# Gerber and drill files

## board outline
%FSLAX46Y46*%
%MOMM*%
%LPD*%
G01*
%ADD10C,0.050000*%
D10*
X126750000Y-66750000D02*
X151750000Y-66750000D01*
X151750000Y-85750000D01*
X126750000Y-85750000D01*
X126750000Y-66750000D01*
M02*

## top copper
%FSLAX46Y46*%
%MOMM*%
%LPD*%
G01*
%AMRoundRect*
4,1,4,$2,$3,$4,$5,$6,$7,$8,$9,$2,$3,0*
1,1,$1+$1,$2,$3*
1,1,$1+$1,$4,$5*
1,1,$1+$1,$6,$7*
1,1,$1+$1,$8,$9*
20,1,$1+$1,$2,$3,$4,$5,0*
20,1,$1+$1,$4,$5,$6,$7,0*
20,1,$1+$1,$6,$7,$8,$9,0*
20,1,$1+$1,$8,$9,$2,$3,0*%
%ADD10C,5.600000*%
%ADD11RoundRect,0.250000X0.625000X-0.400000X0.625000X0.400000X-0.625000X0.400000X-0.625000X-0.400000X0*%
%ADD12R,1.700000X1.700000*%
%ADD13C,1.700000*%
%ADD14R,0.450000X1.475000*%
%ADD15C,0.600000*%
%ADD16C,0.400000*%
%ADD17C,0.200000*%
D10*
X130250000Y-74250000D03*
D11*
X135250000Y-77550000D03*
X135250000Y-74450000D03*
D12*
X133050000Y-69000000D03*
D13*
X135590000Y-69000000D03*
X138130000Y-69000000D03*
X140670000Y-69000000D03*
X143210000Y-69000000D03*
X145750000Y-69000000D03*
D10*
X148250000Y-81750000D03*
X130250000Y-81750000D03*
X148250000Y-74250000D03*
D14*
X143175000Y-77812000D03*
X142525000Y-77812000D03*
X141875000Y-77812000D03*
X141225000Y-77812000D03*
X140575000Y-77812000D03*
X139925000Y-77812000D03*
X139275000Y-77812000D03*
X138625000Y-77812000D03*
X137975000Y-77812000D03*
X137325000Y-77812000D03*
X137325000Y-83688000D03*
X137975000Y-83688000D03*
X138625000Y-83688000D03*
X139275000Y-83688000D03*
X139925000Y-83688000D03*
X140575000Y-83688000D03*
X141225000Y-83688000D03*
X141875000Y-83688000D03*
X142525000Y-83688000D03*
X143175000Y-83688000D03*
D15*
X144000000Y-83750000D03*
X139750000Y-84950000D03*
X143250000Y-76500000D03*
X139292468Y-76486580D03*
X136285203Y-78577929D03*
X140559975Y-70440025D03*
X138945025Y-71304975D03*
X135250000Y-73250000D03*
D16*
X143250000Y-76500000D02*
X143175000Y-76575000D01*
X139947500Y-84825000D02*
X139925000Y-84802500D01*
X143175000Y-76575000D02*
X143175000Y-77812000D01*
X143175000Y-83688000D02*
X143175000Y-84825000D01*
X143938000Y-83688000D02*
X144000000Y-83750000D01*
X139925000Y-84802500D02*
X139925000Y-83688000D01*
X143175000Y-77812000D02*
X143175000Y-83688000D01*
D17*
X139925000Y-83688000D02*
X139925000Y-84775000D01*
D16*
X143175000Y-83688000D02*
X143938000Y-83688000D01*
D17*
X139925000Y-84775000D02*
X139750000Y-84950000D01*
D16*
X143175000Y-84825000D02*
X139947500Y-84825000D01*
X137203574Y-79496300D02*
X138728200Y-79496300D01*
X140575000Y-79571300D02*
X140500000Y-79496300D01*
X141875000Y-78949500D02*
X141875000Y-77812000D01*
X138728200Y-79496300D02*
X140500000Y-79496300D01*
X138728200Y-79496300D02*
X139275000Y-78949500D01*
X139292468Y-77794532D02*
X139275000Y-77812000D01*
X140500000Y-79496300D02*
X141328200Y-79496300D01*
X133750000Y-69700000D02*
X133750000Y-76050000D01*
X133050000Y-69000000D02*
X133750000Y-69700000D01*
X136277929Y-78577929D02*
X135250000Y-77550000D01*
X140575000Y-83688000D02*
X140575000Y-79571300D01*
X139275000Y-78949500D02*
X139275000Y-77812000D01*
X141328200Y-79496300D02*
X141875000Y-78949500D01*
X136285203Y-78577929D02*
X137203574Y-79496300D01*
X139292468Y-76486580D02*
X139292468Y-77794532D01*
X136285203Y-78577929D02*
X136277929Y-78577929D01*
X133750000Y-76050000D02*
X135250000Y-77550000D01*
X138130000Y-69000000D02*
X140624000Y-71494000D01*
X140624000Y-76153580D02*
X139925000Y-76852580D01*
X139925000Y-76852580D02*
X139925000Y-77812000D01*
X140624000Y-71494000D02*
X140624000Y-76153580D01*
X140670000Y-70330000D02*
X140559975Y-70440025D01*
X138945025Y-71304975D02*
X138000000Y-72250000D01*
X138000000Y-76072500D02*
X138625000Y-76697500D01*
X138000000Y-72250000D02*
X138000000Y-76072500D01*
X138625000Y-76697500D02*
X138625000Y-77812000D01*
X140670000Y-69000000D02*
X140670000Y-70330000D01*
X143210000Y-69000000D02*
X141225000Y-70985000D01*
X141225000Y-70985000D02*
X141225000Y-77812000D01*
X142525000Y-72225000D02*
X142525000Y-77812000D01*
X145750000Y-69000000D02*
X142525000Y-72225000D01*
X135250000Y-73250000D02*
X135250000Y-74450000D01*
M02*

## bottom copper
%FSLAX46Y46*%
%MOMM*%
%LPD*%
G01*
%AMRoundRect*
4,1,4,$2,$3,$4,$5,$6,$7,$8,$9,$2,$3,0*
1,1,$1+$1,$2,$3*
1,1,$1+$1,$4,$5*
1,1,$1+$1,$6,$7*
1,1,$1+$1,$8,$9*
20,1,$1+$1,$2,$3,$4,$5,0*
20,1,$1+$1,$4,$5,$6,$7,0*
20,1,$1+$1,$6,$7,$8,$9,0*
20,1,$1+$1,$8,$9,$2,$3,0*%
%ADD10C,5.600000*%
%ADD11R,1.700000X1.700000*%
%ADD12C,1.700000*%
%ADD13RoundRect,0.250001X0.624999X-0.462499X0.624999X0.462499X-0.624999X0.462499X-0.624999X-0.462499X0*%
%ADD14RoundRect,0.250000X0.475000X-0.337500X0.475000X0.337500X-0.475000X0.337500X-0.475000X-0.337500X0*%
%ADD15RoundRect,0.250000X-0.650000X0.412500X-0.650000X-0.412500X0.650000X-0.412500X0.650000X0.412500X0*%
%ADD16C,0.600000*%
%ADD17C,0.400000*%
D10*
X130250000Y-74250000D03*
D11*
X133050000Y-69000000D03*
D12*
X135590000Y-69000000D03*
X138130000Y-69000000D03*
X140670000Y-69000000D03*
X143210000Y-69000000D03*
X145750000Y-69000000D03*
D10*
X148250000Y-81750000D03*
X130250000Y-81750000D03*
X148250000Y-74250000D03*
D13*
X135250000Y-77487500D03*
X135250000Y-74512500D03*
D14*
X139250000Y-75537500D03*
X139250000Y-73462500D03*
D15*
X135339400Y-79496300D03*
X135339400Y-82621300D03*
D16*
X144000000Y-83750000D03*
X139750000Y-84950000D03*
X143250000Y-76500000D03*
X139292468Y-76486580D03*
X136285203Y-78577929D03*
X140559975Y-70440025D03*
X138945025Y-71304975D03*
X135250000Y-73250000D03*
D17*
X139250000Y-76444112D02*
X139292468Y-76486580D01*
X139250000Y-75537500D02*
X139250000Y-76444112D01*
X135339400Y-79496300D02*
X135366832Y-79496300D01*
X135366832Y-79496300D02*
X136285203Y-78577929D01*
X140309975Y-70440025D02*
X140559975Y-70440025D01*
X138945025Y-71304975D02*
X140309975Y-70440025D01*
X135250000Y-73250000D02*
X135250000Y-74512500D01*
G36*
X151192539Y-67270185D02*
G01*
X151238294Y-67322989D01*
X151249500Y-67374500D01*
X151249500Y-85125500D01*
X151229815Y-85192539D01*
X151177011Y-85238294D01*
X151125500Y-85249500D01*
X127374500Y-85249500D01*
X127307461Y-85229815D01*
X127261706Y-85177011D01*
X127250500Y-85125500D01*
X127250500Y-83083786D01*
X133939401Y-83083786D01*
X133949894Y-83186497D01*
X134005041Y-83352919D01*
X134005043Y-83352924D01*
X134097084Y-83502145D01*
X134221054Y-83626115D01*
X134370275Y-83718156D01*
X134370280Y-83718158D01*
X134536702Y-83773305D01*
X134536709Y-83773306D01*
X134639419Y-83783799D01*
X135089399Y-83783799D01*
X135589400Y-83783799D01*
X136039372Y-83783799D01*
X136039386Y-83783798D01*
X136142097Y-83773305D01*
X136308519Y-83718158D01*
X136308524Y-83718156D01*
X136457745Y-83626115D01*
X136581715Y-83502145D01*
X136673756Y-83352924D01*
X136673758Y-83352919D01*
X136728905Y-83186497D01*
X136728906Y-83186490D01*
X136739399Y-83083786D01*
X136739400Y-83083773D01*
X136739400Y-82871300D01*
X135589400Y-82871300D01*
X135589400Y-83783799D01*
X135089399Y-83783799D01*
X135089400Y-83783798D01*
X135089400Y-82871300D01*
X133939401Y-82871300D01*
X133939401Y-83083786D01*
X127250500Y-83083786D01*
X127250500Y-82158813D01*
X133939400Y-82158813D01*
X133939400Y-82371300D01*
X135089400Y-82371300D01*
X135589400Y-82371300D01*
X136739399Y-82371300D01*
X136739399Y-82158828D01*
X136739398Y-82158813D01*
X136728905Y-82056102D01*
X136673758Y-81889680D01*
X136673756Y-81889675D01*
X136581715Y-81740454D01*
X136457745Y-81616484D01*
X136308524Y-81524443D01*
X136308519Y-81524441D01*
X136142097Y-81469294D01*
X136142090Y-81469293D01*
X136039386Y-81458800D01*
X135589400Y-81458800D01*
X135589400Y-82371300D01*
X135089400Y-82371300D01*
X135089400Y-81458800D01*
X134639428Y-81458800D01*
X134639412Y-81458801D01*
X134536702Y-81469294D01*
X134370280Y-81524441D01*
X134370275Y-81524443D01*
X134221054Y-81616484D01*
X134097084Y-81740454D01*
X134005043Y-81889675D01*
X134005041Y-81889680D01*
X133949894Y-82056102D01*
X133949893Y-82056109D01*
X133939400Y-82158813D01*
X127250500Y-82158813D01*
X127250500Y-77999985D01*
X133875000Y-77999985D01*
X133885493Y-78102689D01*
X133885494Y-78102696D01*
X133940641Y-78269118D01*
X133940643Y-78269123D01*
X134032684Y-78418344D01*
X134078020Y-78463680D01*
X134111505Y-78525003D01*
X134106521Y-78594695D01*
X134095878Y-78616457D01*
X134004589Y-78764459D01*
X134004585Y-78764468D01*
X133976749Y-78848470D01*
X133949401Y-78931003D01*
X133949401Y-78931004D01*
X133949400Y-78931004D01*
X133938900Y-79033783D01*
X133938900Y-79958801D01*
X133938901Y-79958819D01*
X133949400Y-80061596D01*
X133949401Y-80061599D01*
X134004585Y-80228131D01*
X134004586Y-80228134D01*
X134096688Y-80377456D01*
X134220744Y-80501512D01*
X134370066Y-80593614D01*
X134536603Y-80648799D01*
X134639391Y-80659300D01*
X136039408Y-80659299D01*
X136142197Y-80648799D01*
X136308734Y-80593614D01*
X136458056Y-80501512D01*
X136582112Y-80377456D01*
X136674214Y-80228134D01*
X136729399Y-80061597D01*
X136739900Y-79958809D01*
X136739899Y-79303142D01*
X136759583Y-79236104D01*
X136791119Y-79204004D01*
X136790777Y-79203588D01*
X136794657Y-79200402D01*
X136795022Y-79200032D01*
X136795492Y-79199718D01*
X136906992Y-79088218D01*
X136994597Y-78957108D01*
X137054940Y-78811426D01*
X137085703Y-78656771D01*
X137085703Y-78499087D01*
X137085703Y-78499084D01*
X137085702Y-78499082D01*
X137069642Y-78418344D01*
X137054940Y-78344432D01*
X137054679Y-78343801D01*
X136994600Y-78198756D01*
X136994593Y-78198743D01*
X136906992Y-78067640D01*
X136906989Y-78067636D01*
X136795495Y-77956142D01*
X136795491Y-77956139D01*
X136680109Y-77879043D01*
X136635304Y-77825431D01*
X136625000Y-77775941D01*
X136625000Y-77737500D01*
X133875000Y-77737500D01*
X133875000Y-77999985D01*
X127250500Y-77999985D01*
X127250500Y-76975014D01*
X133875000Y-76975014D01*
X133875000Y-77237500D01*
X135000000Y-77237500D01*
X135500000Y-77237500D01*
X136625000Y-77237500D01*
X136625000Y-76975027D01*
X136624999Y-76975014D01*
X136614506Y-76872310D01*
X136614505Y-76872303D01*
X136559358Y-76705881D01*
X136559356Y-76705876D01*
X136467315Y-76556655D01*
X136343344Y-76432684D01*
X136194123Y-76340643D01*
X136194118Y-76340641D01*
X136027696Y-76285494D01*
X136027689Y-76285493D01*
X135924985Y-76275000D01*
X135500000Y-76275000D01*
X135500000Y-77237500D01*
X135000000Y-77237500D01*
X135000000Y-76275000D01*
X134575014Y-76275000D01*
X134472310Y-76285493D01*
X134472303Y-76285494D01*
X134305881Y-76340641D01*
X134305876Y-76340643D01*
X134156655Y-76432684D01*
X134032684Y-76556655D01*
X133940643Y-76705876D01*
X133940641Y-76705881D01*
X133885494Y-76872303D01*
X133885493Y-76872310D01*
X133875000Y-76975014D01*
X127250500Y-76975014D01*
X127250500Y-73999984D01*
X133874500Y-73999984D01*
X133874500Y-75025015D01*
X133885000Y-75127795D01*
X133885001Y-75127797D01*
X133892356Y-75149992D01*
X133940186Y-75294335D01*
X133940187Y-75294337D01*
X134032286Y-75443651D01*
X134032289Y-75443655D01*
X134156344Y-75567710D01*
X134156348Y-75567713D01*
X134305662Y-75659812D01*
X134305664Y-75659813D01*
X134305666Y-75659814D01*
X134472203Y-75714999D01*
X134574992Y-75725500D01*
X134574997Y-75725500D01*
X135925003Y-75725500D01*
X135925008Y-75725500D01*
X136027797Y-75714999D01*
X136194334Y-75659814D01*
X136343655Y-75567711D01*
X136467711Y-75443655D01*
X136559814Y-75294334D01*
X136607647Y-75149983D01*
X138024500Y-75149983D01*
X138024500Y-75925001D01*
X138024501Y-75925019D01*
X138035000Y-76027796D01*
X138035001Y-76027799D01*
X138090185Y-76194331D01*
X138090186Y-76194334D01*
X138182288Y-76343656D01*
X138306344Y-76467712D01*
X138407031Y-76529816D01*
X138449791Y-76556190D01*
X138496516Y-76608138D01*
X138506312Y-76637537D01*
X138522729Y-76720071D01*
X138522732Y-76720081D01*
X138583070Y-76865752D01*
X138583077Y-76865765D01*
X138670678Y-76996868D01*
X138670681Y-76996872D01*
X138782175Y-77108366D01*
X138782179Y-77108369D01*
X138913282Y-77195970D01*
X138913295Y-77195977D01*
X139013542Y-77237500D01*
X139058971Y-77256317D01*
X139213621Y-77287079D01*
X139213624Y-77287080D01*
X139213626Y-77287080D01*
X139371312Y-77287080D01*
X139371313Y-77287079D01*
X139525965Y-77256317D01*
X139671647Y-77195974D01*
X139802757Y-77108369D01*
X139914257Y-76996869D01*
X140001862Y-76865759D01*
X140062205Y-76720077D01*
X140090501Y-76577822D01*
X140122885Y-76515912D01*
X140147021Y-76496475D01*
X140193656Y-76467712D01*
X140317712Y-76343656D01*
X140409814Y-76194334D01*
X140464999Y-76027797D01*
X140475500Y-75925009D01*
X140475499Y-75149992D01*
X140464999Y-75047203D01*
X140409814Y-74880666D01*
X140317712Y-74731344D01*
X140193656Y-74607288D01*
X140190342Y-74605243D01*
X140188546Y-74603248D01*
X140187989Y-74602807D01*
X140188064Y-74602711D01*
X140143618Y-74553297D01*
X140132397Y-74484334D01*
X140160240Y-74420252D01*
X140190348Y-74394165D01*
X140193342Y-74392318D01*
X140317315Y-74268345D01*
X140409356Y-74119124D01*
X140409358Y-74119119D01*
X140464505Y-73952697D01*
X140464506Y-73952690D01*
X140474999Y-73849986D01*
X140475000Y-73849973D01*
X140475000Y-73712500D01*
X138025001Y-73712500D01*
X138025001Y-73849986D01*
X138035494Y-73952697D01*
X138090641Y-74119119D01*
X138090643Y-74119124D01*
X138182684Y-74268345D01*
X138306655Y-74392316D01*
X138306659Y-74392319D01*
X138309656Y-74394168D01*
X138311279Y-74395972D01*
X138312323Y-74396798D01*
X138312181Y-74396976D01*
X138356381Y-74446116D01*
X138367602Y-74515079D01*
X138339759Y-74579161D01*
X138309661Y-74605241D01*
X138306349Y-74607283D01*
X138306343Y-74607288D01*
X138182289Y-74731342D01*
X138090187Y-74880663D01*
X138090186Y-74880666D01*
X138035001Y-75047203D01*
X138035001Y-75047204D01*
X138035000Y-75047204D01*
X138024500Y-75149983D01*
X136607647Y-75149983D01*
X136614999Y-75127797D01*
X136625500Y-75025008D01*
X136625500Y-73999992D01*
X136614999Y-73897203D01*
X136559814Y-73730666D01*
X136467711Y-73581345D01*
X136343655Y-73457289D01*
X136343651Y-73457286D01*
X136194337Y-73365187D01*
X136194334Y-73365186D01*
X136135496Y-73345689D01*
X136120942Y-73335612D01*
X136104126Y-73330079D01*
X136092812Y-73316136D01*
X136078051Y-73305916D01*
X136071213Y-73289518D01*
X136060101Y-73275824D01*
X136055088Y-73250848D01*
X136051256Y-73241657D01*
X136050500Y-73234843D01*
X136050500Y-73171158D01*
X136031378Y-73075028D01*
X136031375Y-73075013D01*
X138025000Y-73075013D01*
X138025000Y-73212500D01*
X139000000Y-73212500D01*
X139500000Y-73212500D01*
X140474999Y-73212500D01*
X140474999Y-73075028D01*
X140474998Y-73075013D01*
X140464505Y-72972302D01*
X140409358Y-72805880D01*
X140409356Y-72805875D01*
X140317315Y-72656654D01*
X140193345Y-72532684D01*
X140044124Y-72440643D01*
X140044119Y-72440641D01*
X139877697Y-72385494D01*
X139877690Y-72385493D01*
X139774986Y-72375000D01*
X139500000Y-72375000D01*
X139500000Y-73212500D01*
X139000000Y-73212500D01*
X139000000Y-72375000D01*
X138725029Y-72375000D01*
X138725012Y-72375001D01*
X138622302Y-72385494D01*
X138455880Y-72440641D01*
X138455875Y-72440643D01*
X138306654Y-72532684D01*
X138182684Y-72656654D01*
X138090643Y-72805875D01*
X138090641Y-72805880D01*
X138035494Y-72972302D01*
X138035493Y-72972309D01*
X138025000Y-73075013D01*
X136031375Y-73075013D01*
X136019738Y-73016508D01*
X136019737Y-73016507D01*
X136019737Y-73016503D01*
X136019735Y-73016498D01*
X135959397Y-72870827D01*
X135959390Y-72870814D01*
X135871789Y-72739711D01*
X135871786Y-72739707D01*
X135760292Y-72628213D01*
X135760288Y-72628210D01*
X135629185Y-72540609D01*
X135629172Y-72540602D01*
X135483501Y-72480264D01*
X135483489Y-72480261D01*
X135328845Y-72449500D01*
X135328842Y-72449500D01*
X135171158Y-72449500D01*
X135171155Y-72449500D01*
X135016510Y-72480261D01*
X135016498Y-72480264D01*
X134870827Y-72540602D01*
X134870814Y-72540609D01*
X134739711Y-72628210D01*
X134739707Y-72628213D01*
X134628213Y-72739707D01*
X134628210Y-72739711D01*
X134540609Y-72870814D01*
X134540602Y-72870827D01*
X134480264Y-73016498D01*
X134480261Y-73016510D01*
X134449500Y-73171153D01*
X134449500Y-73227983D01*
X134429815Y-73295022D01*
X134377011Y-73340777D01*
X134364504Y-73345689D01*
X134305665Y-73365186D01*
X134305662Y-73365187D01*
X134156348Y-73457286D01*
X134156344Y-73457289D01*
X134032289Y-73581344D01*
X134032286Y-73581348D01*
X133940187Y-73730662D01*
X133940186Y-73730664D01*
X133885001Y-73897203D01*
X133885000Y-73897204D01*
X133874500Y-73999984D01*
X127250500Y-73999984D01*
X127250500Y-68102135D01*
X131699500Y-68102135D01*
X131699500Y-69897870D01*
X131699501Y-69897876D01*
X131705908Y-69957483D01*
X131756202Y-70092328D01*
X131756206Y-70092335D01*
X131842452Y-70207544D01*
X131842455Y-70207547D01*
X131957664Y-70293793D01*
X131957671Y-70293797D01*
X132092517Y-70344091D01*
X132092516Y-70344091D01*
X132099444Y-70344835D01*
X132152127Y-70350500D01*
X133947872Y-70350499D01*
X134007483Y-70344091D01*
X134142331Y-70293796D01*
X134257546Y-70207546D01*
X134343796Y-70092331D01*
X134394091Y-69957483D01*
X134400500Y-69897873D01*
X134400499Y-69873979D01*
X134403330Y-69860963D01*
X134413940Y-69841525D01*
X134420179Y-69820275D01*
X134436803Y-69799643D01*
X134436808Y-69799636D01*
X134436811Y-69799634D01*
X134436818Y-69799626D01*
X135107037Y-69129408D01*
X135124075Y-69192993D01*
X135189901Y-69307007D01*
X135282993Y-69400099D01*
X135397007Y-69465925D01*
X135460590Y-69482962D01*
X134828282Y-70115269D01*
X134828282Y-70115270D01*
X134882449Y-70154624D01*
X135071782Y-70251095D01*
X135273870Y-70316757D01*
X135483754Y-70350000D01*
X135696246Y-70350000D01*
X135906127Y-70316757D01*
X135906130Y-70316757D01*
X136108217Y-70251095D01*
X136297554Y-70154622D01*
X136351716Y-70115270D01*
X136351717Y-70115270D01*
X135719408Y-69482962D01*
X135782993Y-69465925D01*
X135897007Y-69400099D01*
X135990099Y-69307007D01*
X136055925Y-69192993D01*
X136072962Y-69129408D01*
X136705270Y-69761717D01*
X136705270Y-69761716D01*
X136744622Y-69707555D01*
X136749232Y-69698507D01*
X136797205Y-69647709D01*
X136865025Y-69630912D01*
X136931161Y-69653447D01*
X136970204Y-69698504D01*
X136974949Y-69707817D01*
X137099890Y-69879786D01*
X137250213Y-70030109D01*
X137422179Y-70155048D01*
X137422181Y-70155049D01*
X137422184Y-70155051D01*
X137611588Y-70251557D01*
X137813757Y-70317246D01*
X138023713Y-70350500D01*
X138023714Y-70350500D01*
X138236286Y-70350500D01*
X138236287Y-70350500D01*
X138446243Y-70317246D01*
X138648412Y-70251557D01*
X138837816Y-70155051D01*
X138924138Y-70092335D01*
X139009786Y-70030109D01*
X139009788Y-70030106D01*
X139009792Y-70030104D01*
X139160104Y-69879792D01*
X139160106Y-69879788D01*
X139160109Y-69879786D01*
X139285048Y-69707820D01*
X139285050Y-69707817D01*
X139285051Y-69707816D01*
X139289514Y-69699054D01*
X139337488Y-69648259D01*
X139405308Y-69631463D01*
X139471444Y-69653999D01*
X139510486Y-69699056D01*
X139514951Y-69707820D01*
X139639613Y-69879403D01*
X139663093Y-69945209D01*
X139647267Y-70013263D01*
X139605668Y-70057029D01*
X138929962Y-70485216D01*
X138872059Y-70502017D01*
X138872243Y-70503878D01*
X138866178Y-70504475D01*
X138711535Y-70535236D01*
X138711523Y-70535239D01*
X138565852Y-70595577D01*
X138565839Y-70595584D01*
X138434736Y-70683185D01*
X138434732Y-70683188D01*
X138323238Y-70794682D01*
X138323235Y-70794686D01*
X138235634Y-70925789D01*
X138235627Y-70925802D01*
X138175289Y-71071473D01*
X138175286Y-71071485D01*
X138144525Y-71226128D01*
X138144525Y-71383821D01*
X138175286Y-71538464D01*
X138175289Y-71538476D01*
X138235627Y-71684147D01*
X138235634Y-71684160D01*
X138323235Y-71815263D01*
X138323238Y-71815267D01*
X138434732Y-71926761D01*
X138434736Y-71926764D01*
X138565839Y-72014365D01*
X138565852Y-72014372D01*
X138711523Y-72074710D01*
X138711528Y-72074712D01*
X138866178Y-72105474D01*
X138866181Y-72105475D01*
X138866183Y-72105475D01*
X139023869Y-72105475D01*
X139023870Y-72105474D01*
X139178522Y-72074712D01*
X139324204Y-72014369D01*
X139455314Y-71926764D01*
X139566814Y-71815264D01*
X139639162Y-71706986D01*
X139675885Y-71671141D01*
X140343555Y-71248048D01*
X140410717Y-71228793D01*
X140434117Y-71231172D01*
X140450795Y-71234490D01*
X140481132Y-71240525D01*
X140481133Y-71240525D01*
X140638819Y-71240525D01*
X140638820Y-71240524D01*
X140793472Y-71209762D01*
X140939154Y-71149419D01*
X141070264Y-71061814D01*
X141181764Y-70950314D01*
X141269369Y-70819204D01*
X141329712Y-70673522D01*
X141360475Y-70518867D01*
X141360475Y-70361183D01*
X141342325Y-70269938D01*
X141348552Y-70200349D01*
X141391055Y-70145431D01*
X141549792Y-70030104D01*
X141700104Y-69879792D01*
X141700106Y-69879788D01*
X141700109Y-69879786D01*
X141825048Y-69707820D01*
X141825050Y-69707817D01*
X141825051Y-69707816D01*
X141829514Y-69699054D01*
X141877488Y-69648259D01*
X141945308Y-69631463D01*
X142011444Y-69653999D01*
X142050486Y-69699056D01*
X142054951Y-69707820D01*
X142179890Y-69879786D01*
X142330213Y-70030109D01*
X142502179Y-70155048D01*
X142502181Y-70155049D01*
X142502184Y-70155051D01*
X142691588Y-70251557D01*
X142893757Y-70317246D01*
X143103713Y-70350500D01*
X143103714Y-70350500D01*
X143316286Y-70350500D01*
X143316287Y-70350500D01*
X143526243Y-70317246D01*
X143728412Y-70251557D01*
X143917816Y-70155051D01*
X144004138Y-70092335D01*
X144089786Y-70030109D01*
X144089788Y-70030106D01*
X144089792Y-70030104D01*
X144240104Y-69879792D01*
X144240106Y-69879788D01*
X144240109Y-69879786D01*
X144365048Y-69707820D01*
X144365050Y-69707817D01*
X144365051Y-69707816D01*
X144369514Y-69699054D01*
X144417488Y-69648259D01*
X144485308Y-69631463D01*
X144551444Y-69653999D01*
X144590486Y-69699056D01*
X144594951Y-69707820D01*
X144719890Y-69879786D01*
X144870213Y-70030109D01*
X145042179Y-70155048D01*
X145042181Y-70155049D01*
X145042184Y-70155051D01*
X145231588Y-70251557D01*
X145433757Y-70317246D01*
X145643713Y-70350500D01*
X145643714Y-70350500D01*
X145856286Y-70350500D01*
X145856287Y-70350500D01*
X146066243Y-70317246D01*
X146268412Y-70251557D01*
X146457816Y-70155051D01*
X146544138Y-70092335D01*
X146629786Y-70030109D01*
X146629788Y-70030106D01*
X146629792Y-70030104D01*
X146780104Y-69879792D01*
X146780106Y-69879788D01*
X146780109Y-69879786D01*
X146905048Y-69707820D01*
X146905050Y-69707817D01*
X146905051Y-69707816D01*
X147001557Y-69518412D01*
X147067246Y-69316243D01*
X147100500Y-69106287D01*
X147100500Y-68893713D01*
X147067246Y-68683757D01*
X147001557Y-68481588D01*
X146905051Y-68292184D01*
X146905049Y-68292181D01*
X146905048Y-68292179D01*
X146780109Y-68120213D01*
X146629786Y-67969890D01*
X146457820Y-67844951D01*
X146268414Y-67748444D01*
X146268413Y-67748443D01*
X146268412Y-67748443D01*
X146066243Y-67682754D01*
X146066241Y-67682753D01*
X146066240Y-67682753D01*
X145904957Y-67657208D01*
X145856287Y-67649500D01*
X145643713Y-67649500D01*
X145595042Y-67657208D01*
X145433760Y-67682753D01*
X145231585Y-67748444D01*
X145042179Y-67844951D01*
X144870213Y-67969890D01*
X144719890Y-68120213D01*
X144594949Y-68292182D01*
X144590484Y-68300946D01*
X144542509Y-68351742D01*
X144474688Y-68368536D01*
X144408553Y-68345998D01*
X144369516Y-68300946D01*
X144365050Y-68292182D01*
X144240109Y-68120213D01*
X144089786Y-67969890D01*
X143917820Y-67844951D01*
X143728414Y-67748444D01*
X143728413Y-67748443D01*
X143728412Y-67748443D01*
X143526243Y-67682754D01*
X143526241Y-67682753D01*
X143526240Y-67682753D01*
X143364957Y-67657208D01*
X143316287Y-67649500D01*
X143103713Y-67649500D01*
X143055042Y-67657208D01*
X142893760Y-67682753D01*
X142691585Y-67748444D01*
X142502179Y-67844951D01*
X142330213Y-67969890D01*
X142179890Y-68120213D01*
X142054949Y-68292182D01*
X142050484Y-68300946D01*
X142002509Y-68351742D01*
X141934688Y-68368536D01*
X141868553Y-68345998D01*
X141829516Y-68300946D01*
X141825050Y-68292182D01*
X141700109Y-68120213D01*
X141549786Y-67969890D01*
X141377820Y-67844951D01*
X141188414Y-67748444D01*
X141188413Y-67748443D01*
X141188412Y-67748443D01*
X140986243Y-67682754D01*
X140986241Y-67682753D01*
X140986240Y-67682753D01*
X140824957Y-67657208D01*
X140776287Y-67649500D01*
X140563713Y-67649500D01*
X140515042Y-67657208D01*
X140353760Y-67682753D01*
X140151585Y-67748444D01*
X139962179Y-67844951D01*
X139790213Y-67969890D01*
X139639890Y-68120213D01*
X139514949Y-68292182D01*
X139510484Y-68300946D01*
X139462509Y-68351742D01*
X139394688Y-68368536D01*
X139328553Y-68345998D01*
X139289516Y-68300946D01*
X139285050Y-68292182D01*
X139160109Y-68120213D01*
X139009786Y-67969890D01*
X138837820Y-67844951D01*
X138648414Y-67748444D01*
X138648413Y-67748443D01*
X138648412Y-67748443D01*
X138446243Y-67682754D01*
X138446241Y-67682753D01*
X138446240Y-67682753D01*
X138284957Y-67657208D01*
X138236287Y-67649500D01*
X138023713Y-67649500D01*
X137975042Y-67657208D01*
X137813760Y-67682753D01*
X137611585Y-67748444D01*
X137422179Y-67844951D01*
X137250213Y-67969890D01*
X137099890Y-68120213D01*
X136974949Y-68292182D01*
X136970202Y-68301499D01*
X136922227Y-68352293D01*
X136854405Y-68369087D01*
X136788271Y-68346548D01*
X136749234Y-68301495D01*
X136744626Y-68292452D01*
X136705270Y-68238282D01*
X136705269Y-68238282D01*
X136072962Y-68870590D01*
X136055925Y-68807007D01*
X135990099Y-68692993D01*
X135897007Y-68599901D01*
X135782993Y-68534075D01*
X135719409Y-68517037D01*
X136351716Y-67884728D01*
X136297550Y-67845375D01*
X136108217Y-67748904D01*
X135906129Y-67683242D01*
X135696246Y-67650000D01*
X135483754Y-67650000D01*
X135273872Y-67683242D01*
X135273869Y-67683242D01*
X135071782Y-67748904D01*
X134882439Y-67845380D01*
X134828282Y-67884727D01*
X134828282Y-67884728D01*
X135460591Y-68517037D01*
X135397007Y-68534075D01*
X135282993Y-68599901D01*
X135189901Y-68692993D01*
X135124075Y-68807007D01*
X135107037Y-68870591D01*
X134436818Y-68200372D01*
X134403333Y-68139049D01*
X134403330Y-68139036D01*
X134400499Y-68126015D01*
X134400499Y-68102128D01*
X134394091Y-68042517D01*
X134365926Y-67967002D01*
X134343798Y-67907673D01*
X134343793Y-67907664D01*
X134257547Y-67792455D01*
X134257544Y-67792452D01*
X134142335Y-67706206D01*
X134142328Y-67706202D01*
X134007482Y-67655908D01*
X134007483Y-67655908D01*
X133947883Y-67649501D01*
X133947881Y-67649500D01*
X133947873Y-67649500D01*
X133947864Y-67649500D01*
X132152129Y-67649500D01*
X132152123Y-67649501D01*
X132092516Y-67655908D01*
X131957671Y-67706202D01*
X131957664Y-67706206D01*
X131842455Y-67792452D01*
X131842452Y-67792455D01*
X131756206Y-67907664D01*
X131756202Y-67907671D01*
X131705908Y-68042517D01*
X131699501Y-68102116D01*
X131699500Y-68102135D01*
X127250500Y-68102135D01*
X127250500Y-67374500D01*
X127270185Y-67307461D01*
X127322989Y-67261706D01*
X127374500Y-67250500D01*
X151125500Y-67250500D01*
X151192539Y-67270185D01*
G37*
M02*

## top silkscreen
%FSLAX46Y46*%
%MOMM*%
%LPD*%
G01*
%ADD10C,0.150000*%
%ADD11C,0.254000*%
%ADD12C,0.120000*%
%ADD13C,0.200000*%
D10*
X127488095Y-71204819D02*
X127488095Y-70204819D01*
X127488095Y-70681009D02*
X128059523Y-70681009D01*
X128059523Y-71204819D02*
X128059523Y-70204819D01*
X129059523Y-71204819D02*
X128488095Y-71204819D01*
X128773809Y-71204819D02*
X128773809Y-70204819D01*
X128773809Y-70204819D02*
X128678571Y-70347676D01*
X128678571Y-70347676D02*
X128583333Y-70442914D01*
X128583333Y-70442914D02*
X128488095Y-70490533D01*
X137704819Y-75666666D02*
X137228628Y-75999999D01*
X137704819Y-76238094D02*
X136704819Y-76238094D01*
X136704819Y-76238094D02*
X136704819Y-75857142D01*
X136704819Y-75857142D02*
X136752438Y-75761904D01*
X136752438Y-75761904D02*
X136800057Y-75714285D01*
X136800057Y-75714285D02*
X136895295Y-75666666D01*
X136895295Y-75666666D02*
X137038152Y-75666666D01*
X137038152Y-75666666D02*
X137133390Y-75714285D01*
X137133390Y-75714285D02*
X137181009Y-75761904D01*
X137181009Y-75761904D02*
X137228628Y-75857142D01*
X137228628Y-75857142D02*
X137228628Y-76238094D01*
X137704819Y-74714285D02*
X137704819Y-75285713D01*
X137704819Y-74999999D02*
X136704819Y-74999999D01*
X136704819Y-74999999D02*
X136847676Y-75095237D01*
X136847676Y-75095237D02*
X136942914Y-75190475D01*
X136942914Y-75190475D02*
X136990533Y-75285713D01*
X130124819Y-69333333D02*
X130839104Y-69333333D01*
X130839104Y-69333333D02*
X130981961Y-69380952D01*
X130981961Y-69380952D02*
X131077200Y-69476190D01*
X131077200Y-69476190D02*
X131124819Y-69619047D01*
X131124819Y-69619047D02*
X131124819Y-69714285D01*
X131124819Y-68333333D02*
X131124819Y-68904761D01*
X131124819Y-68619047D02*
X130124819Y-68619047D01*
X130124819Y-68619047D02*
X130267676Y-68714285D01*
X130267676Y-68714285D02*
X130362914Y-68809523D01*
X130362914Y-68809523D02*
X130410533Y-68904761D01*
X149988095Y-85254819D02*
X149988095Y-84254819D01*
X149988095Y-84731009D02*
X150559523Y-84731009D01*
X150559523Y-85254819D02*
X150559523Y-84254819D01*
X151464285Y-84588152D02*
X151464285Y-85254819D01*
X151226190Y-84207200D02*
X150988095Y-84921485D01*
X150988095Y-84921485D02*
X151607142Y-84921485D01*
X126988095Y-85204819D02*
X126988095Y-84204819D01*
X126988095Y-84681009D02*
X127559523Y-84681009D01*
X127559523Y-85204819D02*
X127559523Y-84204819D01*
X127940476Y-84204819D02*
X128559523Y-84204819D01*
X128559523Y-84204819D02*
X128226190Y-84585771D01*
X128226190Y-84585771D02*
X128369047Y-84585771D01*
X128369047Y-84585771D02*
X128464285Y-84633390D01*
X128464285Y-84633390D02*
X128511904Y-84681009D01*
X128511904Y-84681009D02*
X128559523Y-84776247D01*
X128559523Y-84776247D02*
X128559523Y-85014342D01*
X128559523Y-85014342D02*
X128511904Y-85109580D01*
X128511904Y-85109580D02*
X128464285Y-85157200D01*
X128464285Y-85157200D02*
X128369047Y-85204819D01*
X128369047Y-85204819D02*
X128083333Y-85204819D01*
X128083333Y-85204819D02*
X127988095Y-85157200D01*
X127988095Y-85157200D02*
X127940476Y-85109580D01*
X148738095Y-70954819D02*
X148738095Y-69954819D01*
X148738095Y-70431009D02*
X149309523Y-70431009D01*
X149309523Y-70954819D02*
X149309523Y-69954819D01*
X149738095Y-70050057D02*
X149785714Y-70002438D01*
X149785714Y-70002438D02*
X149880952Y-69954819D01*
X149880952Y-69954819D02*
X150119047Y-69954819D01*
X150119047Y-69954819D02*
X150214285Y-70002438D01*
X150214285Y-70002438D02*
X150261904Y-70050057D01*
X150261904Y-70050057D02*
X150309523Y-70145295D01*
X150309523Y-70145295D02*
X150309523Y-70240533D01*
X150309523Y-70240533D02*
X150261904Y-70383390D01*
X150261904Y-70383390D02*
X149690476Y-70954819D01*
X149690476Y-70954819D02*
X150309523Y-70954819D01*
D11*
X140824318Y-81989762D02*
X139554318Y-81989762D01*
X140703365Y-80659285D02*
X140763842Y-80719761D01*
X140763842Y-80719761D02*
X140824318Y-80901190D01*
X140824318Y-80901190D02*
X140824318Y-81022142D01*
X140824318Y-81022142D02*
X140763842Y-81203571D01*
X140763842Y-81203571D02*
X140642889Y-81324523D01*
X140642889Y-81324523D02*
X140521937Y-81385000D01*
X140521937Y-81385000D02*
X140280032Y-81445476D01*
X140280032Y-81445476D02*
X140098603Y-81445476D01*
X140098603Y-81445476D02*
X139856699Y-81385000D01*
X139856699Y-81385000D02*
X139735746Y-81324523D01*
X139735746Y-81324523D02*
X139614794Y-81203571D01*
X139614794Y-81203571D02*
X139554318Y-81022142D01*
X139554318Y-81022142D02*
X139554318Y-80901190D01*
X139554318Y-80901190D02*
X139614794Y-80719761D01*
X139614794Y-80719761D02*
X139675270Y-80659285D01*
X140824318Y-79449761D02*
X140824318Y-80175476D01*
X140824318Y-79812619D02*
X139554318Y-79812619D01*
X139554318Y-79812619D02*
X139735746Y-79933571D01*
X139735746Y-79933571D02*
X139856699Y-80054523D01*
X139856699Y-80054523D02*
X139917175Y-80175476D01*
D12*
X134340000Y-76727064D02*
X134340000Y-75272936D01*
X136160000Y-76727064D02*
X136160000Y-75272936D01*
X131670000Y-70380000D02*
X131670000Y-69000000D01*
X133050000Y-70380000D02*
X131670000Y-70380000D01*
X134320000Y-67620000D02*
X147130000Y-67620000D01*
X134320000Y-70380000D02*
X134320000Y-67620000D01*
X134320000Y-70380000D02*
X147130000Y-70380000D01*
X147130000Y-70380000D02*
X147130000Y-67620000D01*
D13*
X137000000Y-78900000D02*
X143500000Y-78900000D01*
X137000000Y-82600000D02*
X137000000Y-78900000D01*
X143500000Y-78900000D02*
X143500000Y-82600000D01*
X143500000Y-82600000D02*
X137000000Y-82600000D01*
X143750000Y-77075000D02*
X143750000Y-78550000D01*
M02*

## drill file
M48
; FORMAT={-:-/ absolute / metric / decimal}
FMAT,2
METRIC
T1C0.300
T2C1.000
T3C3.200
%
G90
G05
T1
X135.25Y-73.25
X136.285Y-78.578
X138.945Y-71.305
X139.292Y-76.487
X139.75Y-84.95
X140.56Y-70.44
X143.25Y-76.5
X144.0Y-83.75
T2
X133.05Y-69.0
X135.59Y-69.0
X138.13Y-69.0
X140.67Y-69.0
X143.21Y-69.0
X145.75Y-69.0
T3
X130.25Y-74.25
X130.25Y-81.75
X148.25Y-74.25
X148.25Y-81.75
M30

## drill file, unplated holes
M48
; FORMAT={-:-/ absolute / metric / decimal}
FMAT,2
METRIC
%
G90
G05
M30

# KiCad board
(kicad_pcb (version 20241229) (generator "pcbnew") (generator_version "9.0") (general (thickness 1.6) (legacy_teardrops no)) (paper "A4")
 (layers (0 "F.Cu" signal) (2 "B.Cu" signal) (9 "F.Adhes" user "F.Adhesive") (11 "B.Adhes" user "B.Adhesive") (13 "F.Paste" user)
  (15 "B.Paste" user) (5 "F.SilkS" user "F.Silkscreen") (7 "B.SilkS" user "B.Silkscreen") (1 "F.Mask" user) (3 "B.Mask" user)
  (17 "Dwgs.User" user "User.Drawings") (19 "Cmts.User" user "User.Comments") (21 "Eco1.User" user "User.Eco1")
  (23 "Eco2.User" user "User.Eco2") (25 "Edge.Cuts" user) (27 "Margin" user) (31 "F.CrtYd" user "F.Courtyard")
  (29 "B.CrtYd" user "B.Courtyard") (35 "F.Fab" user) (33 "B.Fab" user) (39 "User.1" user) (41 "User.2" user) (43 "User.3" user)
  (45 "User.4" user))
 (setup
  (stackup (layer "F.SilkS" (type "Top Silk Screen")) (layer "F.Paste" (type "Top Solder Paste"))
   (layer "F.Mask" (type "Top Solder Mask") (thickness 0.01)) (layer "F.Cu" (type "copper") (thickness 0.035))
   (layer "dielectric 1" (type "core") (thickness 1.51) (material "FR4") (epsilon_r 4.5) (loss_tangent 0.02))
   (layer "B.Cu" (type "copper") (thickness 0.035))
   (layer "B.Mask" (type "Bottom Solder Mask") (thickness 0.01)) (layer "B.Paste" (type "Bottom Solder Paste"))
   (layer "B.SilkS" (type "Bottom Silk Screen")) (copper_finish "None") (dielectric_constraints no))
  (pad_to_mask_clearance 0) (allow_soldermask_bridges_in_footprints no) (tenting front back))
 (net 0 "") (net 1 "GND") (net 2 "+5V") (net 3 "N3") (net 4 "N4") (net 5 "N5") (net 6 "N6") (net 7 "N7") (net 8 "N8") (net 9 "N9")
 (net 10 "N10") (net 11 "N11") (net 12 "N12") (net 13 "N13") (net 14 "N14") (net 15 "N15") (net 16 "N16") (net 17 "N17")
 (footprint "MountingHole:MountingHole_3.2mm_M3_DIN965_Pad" (layer "F.Cu") (at 130.25 74.25)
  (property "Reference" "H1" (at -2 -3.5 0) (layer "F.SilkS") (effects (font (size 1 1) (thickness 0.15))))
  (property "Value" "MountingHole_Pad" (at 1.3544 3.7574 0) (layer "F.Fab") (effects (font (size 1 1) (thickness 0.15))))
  (pad "1" thru_hole circle (at 0 0) (size 5.6 5.6) (drill 3.2) (layers "*.Cu" "*.Mask") (remove_unused_layers no) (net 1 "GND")
   (zone_connect 2)))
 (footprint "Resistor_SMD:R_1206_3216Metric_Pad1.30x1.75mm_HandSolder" (layer "F.Cu") (at 135.25 76 90)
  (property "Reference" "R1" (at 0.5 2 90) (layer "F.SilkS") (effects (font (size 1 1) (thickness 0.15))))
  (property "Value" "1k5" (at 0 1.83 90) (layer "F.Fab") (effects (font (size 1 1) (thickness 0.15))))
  (fp_line (start -0.727064 -0.91) (end 0.727064 -0.91) (stroke (width 0.12) (type solid)) (layer "F.SilkS"))
  (fp_line (start -0.727064 0.91) (end 0.727064 0.91) (stroke (width 0.12) (type solid)) (layer "F.SilkS"))
  (pad "1" smd roundrect (at -1.55 0 90) (size 1.3 1.75) (layers "F.Cu" "F.Mask" "F.Paste") (roundrect_rratio 0.192308) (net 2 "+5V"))
  (pad "2" smd roundrect (at 1.55 0 90) (size 1.3 1.75) (layers "F.Cu" "F.Mask" "F.Paste") (roundrect_rratio 0.192308) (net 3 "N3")))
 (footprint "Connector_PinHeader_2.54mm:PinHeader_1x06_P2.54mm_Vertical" (layer "F.Cu") (at 133.05 69 90)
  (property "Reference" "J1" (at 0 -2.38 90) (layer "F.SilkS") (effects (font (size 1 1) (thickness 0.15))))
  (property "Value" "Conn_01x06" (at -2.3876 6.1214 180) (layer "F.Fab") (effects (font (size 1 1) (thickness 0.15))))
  (fp_line (start -1.38 -1.38) (end 0 -1.38) (stroke (width 0.12) (type solid)) (layer "F.SilkS"))
  (fp_line (start -1.38 0) (end -1.38 -1.38) (stroke (width 0.12) (type solid)) (layer "F.SilkS"))
  (fp_line (start 1.38 1.27) (end 1.38 14.08) (stroke (width 0.12) (type solid)) (layer "F.SilkS"))
  (fp_line (start -1.38 1.27) (end 1.38 1.27) (stroke (width 0.12) (type solid)) (layer "F.SilkS"))
  (fp_line (start -1.38 1.27) (end -1.38 14.08) (stroke (width 0.12) (type solid)) (layer "F.SilkS"))
  (fp_line (start -1.38 14.08) (end 1.38 14.08) (stroke (width 0.12) (type solid)) (layer "F.SilkS"))
  (pad "1" thru_hole rect (at 0 0 90) (size 1.7 1.7) (drill 1) (layers "*.Cu" "*.Mask") (remove_unused_layers no) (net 2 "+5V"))
  (pad "2" thru_hole circle (at 0 2.54 90) (size 1.7 1.7) (drill 1) (layers "*.Cu" "*.Mask") (remove_unused_layers no) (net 1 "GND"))
  (pad "3" thru_hole circle (at 0 5.08 90) (size 1.7 1.7) (drill 1) (layers "*.Cu" "*.Mask") (remove_unused_layers no) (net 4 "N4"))
  (pad "4" thru_hole circle (at 0 7.62 90) (size 1.7 1.7) (drill 1) (layers "*.Cu" "*.Mask") (remove_unused_layers no) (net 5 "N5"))
  (pad "5" thru_hole circle (at 0 10.16 90) (size 1.7 1.7) (drill 1) (layers "*.Cu" "*.Mask") (remove_unused_layers no) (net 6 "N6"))
  (pad "6" thru_hole circle (at 0 12.7 90) (size 1.7 1.7) (drill 1) (layers "*.Cu" "*.Mask") (remove_unused_layers no) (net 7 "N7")))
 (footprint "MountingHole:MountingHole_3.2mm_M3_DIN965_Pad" (layer "F.Cu") (at 148.25 81.75)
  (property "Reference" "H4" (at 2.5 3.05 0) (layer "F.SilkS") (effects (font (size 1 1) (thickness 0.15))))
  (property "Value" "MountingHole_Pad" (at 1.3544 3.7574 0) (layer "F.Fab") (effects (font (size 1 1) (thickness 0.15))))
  (pad "1" thru_hole circle (at 0 0) (size 5.6 5.6) (drill 3.2) (layers "*.Cu" "*.Mask") (remove_unused_layers no) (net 1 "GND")
   (zone_connect 2)))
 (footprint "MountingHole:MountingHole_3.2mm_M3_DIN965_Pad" (layer "F.Cu") (at 130.25 81.75)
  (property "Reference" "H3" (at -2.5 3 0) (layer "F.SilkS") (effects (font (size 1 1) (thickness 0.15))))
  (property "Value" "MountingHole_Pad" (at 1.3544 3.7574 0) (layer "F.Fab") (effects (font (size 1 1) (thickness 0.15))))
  (pad "1" thru_hole circle (at 0 0) (size 5.6 5.6) (drill 3.2) (layers "*.Cu" "*.Mask") (remove_unused_layers no) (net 1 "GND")
   (zone_connect 2)))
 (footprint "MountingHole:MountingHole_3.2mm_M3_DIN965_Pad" (layer "F.Cu") (at 148.25 74.25)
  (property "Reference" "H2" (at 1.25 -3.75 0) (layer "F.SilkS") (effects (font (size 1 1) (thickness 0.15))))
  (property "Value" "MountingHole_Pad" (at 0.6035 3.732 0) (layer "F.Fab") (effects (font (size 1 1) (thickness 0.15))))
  (pad "1" thru_hole circle (at 0 0) (size 5.6 5.6) (drill 3.2) (layers "*.Cu" "*.Mask") (remove_unused_layers no) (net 1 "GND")
   (zone_connect 2)))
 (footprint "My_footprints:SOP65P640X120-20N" (layer "F.Cu") (at 140.25 80.75 -90)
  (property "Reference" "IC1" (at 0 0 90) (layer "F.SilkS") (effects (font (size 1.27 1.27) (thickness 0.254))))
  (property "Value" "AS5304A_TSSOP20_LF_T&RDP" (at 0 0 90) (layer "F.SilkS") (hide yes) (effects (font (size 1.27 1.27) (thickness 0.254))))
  (fp_line (start -1.85 3.25) (end -1.85 -3.25) (stroke (width 0.2) (type solid)) (layer "F.SilkS"))
  (fp_line (start 1.85 3.25) (end -1.85 3.25) (stroke (width 0.2) (type solid)) (layer "F.SilkS"))
  (fp_line (start -1.85 -3.25) (end 1.85 -3.25) (stroke (width 0.2) (type solid)) (layer "F.SilkS"))
  (fp_line (start 1.85 -3.25) (end 1.85 3.25) (stroke (width 0.2) (type solid)) (layer "F.SilkS"))
  (fp_line (start -3.675 -3.5) (end -2.2 -3.5) (stroke (width 0.2) (type solid)) (layer "F.SilkS"))
  (pad "1" smd rect (at -2.938 -2.925) (size 0.45 1.475) (layers "F.Cu" "F.Mask" "F.Paste") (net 1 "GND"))
  (pad "2" smd rect (at -2.938 -2.275) (size 0.45 1.475) (layers "F.Cu" "F.Mask" "F.Paste") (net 7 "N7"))
  (pad "3" smd rect (at -2.938 -1.625) (size 0.45 1.475) (layers "F.Cu" "F.Mask" "F.Paste") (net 2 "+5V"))
  (pad "4" smd rect (at -2.938 -0.975) (size 0.45 1.475) (layers "F.Cu" "F.Mask" "F.Paste") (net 6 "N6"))
  (pad "5" smd rect (at -2.938 -0.325) (size 0.45 1.475) (layers "F.Cu" "F.Mask" "F.Paste") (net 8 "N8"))
  (pad "6" smd rect (at -2.938 0.325) (size 0.45 1.475) (layers "F.Cu" "F.Mask" "F.Paste") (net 4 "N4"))
  (pad "7" smd rect (at -2.938 0.975) (size 0.45 1.475) (layers "F.Cu" "F.Mask" "F.Paste") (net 2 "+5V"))
  (pad "8" smd rect (at -2.938 1.625) (size 0.45 1.475) (layers "F.Cu" "F.Mask" "F.Paste") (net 5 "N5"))
  (pad "9" smd rect (at -2.938 2.275) (size 0.45 1.475) (layers "F.Cu" "F.Mask" "F.Paste") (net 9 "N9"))
  (pad "10" smd rect (at -2.938 2.925) (size 0.45 1.475) (layers "F.Cu" "F.Mask" "F.Paste") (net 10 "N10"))
  (pad "11" smd rect (at 2.938 2.925) (size 0.45 1.475) (layers "F.Cu" "F.Mask" "F.Paste") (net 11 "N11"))
  (pad "12" smd rect (at 2.938 2.275) (size 0.45 1.475) (layers "F.Cu" "F.Mask" "F.Paste") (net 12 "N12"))
  (pad "13" smd rect (at 2.938 1.625) (size 0.45 1.475) (layers "F.Cu" "F.Mask" "F.Paste") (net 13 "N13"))
  (pad "14" smd rect (at 2.938 0.975) (size 0.45 1.475) (layers "F.Cu" "F.Mask" "F.Paste") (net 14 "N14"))
  (pad "15" smd rect (at 2.938 0.325) (size 0.45 1.475) (layers "F.Cu" "F.Mask" "F.Paste") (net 1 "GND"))
  (pad "16" smd rect (at 2.938 -0.325) (size 0.45 1.475) (layers "F.Cu" "F.Mask" "F.Paste") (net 2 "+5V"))
  (pad "17" smd rect (at 2.938 -0.975) (size 0.45 1.475) (layers "F.Cu" "F.Mask" "F.Paste") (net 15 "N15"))
  (pad "18" smd rect (at 2.938 -1.625) (size 0.45 1.475) (layers "F.Cu" "F.Mask" "F.Paste") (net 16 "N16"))
  (pad "19" smd rect (at 2.938 -2.275) (size 0.45 1.475) (layers "F.Cu" "F.Mask" "F.Paste") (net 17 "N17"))
  (pad "20" smd rect (at 2.938 -2.925) (size 0.45 1.475) (layers "F.Cu" "F.Mask" "F.Paste") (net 1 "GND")))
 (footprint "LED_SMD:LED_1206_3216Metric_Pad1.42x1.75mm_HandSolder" (layer "B.Cu") (at 135.25 76 90)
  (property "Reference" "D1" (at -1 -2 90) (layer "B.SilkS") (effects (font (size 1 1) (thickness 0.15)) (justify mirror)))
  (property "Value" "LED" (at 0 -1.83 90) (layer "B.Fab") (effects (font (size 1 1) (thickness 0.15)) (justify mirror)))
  (pad "1" smd roundrect (at -1.4875 0 90) (size 1.425 1.75) (layers "B.Cu" "B.Mask" "B.Paste") (roundrect_rratio 0.175439) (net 1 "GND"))
  (pad "2" smd roundrect (at 1.4875 0 90) (size 1.425 1.75) (layers "B.Cu" "B.Mask" "B.Paste") (roundrect_rratio 0.175439) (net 3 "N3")))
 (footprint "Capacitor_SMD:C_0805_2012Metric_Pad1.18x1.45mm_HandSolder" (layer "B.Cu") (at 139.25 74.5 90)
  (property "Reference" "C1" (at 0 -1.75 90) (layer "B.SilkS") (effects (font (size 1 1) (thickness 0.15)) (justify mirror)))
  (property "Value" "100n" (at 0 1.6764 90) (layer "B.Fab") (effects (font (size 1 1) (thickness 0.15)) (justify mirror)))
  (pad "1" smd roundrect (at -1.0375 0 90) (size 1.175 1.45) (layers "B.Cu" "B.Mask" "B.Paste") (roundrect_rratio 0.212766) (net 2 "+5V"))
  (pad "2" smd roundrect (at 1.0375 0 90) (size 1.175 1.45) (layers "B.Cu" "B.Mask" "B.Paste") (roundrect_rratio 0.212766) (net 1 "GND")))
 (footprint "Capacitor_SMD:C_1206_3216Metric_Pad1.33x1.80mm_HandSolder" (layer "B.Cu") (at 135.3394 81.0588 -90)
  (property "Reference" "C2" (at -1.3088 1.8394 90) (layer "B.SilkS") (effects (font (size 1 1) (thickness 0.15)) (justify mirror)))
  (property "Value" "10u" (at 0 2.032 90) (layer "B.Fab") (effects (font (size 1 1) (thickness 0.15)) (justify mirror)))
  (pad "1" smd roundrect (at -1.5625 0 270) (size 1.325 1.8) (layers "B.Cu" "B.Mask" "B.Paste") (roundrect_rratio 0.188679) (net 2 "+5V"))
  (pad "2" smd roundrect (at 1.5625 0 270) (size 1.325 1.8) (layers "B.Cu" "B.Mask" "B.Paste") (roundrect_rratio 0.188679) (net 1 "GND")))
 (gr_rect (start 126.75 66.75) (end 151.75 85.75) (stroke (width 0.05) (type default)) (fill no) (layer "Edge.Cuts"))
 (segment (start 143.25 76.5) (end 143.175 76.575) (width 0.4) (layer "F.Cu") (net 1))
 (segment (start 139.9475 84.825) (end 139.925 84.8025) (width 0.4) (layer "F.Cu") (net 1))
 (segment (start 143.175 76.575) (end 143.175 77.812) (width 0.4) (layer "F.Cu") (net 1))
 (segment (start 143.175 83.688) (end 143.175 84.825) (width 0.4) (layer "F.Cu") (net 1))
 (segment (start 143.938 83.688) (end 144 83.75) (width 0.4) (layer "F.Cu") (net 1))
 (segment (start 139.925 84.8025) (end 139.925 83.688) (width 0.4) (layer "F.Cu") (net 1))
 (segment (start 143.175 77.812) (end 143.175 83.688) (width 0.4) (layer "F.Cu") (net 1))
 (segment (start 139.925 83.688) (end 139.925 84.775) (width 0.2) (layer "F.Cu") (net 1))
 (segment (start 143.175 83.688) (end 143.938 83.688) (width 0.4) (layer "F.Cu") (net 1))
 (segment (start 139.925 84.775) (end 139.75 84.95) (width 0.2) (layer "F.Cu") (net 1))
 (segment (start 143.175 84.825) (end 139.9475 84.825) (width 0.4) (layer "F.Cu") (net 1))
 (via (at 144 83.75) (size 0.6) (drill 0.3) (layers "F.Cu" "B.Cu") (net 1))
 (via (at 139.75 84.95) (size 0.6) (drill 0.3) (layers "F.Cu" "B.Cu") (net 1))
 (via (at 143.25 76.5) (size 0.6) (drill 0.3) (layers "F.Cu" "B.Cu") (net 1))
 (segment (start 137.203574 79.4963) (end 138.7282 79.4963) (width 0.4) (layer "F.Cu") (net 2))
 (segment (start 140.575 79.5713) (end 140.5 79.4963) (width 0.4) (layer "F.Cu") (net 2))
 (segment (start 141.875 78.9495) (end 141.875 77.812) (width 0.4) (layer "F.Cu") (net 2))
 (segment (start 138.7282 79.4963) (end 140.5 79.4963) (width 0.4) (layer "F.Cu") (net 2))
 (segment (start 138.7282 79.4963) (end 139.275 78.9495) (width 0.4) (layer "F.Cu") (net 2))
 (segment (start 139.292468 77.794532) (end 139.275 77.812) (width 0.4) (layer "F.Cu") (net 2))
 (segment (start 140.5 79.4963) (end 141.3282 79.4963) (width 0.4) (layer "F.Cu") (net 2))
 (segment (start 133.75 69.7) (end 133.75 76.05) (width 0.4) (layer "F.Cu") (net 2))
 (segment (start 133.05 69) (end 133.75 69.7) (width 0.4) (layer "F.Cu") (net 2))
 (segment (start 136.277929 78.577929) (end 135.25 77.55) (width 0.4) (layer "F.Cu") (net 2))
 (segment (start 140.575 83.688) (end 140.575 79.5713) (width 0.4) (layer "F.Cu") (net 2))
 (segment (start 139.275 78.9495) (end 139.275 77.812) (width 0.4) (layer "F.Cu") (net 2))
 (segment (start 141.3282 79.4963) (end 141.875 78.9495) (width 0.4) (layer "F.Cu") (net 2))
 (segment (start 136.285203 78.577929) (end 137.203574 79.4963) (width 0.4) (layer "F.Cu") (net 2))
 (segment (start 139.292468 76.48658) (end 139.292468 77.794532) (width 0.4) (layer "F.Cu") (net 2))
 (segment (start 136.285203 78.577929) (end 136.277929 78.577929) (width 0.4) (layer "F.Cu") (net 2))
 (segment (start 133.75 76.05) (end 135.25 77.55) (width 0.4) (layer "F.Cu") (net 2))
 (via (at 139.292468 76.48658) (size 0.6) (drill 0.3) (layers "F.Cu" "B.Cu") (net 2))
 (via (at 136.285203 78.577929) (size 0.6) (drill 0.3) (layers "F.Cu" "B.Cu") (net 2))
 (segment (start 139.25 76.444112) (end 139.292468 76.48658) (width 0.4) (layer "B.Cu") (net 2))
 (segment (start 139.25 75.5375) (end 139.25 76.444112) (width 0.4) (layer "B.Cu") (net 2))
 (segment (start 135.3394 79.4963) (end 135.366832 79.4963) (width 0.4) (layer "B.Cu") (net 2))
 (segment (start 135.366832 79.4963) (end 136.285203 78.577929) (width 0.4) (layer "B.Cu") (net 2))
 (segment (start 138.13 69) (end 140.624 71.494) (width 0.4) (layer "F.Cu") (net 4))
 (segment (start 140.624 76.15358) (end 139.925 76.85258) (width 0.4) (layer "F.Cu") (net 4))
 (segment (start 139.925 76.85258) (end 139.925 77.812) (width 0.4) (layer "F.Cu") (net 4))
 (segment (start 140.624 71.494) (end 140.624 76.15358) (width 0.4) (layer "F.Cu") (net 4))
 (segment (start 140.67 70.33) (end 140.559975 70.440025) (width 0.4) (layer "F.Cu") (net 5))
 (segment (start 138.945025 71.304975) (end 138 72.25) (width 0.4) (layer "F.Cu") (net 5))
 (segment (start 138 76.0725) (end 138.625 76.6975) (width 0.4) (layer "F.Cu") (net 5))
 (segment (start 138 72.25) (end 138 76.0725) (width 0.4) (layer "F.Cu") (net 5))
 (segment (start 138.625 76.6975) (end 138.625 77.812) (width 0.4) (layer "F.Cu") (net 5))
 (segment (start 140.67 69) (end 140.67 70.33) (width 0.4) (layer "F.Cu") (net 5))
 (via (at 140.559975 70.440025) (size 0.6) (drill 0.3) (layers "F.Cu" "B.Cu") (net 5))
 (via (at 138.945025 71.304975) (size 0.6) (drill 0.3) (layers "F.Cu" "B.Cu") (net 5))
 (segment (start 140.309975 70.440025) (end 140.559975 70.440025) (width 0.4) (layer "B.Cu") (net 5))
 (segment (start 138.945025 71.304975) (end 140.309975 70.440025) (width 0.4) (layer "B.Cu") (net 5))
 (segment (start 143.21 69) (end 141.225 70.985) (width 0.4) (layer "F.Cu") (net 6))
 (segment (start 141.225 70.985) (end 141.225 77.812) (width 0.4) (layer "F.Cu") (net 6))
 (segment (start 142.525 72.225) (end 142.525 77.812) (width 0.4) (layer "F.Cu") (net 7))
 (segment (start 145.75 69) (end 142.525 72.225) (width 0.4) (layer "F.Cu") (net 7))
 (segment (start 135.25 73.25) (end 135.25 74.45) (width 0.4) (layer "F.Cu") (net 3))
 (via (at 135.25 73.25) (size 0.6) (drill 0.3) (layers "F.Cu" "B.Cu") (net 3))
 (segment (start 135.25 73.25) (end 135.25 74.5125) (width 0.4) (layer "B.Cu") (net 3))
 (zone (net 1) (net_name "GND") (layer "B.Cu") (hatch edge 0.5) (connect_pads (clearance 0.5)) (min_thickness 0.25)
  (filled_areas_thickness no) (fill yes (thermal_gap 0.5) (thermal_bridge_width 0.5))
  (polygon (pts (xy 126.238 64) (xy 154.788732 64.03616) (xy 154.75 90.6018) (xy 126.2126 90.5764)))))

